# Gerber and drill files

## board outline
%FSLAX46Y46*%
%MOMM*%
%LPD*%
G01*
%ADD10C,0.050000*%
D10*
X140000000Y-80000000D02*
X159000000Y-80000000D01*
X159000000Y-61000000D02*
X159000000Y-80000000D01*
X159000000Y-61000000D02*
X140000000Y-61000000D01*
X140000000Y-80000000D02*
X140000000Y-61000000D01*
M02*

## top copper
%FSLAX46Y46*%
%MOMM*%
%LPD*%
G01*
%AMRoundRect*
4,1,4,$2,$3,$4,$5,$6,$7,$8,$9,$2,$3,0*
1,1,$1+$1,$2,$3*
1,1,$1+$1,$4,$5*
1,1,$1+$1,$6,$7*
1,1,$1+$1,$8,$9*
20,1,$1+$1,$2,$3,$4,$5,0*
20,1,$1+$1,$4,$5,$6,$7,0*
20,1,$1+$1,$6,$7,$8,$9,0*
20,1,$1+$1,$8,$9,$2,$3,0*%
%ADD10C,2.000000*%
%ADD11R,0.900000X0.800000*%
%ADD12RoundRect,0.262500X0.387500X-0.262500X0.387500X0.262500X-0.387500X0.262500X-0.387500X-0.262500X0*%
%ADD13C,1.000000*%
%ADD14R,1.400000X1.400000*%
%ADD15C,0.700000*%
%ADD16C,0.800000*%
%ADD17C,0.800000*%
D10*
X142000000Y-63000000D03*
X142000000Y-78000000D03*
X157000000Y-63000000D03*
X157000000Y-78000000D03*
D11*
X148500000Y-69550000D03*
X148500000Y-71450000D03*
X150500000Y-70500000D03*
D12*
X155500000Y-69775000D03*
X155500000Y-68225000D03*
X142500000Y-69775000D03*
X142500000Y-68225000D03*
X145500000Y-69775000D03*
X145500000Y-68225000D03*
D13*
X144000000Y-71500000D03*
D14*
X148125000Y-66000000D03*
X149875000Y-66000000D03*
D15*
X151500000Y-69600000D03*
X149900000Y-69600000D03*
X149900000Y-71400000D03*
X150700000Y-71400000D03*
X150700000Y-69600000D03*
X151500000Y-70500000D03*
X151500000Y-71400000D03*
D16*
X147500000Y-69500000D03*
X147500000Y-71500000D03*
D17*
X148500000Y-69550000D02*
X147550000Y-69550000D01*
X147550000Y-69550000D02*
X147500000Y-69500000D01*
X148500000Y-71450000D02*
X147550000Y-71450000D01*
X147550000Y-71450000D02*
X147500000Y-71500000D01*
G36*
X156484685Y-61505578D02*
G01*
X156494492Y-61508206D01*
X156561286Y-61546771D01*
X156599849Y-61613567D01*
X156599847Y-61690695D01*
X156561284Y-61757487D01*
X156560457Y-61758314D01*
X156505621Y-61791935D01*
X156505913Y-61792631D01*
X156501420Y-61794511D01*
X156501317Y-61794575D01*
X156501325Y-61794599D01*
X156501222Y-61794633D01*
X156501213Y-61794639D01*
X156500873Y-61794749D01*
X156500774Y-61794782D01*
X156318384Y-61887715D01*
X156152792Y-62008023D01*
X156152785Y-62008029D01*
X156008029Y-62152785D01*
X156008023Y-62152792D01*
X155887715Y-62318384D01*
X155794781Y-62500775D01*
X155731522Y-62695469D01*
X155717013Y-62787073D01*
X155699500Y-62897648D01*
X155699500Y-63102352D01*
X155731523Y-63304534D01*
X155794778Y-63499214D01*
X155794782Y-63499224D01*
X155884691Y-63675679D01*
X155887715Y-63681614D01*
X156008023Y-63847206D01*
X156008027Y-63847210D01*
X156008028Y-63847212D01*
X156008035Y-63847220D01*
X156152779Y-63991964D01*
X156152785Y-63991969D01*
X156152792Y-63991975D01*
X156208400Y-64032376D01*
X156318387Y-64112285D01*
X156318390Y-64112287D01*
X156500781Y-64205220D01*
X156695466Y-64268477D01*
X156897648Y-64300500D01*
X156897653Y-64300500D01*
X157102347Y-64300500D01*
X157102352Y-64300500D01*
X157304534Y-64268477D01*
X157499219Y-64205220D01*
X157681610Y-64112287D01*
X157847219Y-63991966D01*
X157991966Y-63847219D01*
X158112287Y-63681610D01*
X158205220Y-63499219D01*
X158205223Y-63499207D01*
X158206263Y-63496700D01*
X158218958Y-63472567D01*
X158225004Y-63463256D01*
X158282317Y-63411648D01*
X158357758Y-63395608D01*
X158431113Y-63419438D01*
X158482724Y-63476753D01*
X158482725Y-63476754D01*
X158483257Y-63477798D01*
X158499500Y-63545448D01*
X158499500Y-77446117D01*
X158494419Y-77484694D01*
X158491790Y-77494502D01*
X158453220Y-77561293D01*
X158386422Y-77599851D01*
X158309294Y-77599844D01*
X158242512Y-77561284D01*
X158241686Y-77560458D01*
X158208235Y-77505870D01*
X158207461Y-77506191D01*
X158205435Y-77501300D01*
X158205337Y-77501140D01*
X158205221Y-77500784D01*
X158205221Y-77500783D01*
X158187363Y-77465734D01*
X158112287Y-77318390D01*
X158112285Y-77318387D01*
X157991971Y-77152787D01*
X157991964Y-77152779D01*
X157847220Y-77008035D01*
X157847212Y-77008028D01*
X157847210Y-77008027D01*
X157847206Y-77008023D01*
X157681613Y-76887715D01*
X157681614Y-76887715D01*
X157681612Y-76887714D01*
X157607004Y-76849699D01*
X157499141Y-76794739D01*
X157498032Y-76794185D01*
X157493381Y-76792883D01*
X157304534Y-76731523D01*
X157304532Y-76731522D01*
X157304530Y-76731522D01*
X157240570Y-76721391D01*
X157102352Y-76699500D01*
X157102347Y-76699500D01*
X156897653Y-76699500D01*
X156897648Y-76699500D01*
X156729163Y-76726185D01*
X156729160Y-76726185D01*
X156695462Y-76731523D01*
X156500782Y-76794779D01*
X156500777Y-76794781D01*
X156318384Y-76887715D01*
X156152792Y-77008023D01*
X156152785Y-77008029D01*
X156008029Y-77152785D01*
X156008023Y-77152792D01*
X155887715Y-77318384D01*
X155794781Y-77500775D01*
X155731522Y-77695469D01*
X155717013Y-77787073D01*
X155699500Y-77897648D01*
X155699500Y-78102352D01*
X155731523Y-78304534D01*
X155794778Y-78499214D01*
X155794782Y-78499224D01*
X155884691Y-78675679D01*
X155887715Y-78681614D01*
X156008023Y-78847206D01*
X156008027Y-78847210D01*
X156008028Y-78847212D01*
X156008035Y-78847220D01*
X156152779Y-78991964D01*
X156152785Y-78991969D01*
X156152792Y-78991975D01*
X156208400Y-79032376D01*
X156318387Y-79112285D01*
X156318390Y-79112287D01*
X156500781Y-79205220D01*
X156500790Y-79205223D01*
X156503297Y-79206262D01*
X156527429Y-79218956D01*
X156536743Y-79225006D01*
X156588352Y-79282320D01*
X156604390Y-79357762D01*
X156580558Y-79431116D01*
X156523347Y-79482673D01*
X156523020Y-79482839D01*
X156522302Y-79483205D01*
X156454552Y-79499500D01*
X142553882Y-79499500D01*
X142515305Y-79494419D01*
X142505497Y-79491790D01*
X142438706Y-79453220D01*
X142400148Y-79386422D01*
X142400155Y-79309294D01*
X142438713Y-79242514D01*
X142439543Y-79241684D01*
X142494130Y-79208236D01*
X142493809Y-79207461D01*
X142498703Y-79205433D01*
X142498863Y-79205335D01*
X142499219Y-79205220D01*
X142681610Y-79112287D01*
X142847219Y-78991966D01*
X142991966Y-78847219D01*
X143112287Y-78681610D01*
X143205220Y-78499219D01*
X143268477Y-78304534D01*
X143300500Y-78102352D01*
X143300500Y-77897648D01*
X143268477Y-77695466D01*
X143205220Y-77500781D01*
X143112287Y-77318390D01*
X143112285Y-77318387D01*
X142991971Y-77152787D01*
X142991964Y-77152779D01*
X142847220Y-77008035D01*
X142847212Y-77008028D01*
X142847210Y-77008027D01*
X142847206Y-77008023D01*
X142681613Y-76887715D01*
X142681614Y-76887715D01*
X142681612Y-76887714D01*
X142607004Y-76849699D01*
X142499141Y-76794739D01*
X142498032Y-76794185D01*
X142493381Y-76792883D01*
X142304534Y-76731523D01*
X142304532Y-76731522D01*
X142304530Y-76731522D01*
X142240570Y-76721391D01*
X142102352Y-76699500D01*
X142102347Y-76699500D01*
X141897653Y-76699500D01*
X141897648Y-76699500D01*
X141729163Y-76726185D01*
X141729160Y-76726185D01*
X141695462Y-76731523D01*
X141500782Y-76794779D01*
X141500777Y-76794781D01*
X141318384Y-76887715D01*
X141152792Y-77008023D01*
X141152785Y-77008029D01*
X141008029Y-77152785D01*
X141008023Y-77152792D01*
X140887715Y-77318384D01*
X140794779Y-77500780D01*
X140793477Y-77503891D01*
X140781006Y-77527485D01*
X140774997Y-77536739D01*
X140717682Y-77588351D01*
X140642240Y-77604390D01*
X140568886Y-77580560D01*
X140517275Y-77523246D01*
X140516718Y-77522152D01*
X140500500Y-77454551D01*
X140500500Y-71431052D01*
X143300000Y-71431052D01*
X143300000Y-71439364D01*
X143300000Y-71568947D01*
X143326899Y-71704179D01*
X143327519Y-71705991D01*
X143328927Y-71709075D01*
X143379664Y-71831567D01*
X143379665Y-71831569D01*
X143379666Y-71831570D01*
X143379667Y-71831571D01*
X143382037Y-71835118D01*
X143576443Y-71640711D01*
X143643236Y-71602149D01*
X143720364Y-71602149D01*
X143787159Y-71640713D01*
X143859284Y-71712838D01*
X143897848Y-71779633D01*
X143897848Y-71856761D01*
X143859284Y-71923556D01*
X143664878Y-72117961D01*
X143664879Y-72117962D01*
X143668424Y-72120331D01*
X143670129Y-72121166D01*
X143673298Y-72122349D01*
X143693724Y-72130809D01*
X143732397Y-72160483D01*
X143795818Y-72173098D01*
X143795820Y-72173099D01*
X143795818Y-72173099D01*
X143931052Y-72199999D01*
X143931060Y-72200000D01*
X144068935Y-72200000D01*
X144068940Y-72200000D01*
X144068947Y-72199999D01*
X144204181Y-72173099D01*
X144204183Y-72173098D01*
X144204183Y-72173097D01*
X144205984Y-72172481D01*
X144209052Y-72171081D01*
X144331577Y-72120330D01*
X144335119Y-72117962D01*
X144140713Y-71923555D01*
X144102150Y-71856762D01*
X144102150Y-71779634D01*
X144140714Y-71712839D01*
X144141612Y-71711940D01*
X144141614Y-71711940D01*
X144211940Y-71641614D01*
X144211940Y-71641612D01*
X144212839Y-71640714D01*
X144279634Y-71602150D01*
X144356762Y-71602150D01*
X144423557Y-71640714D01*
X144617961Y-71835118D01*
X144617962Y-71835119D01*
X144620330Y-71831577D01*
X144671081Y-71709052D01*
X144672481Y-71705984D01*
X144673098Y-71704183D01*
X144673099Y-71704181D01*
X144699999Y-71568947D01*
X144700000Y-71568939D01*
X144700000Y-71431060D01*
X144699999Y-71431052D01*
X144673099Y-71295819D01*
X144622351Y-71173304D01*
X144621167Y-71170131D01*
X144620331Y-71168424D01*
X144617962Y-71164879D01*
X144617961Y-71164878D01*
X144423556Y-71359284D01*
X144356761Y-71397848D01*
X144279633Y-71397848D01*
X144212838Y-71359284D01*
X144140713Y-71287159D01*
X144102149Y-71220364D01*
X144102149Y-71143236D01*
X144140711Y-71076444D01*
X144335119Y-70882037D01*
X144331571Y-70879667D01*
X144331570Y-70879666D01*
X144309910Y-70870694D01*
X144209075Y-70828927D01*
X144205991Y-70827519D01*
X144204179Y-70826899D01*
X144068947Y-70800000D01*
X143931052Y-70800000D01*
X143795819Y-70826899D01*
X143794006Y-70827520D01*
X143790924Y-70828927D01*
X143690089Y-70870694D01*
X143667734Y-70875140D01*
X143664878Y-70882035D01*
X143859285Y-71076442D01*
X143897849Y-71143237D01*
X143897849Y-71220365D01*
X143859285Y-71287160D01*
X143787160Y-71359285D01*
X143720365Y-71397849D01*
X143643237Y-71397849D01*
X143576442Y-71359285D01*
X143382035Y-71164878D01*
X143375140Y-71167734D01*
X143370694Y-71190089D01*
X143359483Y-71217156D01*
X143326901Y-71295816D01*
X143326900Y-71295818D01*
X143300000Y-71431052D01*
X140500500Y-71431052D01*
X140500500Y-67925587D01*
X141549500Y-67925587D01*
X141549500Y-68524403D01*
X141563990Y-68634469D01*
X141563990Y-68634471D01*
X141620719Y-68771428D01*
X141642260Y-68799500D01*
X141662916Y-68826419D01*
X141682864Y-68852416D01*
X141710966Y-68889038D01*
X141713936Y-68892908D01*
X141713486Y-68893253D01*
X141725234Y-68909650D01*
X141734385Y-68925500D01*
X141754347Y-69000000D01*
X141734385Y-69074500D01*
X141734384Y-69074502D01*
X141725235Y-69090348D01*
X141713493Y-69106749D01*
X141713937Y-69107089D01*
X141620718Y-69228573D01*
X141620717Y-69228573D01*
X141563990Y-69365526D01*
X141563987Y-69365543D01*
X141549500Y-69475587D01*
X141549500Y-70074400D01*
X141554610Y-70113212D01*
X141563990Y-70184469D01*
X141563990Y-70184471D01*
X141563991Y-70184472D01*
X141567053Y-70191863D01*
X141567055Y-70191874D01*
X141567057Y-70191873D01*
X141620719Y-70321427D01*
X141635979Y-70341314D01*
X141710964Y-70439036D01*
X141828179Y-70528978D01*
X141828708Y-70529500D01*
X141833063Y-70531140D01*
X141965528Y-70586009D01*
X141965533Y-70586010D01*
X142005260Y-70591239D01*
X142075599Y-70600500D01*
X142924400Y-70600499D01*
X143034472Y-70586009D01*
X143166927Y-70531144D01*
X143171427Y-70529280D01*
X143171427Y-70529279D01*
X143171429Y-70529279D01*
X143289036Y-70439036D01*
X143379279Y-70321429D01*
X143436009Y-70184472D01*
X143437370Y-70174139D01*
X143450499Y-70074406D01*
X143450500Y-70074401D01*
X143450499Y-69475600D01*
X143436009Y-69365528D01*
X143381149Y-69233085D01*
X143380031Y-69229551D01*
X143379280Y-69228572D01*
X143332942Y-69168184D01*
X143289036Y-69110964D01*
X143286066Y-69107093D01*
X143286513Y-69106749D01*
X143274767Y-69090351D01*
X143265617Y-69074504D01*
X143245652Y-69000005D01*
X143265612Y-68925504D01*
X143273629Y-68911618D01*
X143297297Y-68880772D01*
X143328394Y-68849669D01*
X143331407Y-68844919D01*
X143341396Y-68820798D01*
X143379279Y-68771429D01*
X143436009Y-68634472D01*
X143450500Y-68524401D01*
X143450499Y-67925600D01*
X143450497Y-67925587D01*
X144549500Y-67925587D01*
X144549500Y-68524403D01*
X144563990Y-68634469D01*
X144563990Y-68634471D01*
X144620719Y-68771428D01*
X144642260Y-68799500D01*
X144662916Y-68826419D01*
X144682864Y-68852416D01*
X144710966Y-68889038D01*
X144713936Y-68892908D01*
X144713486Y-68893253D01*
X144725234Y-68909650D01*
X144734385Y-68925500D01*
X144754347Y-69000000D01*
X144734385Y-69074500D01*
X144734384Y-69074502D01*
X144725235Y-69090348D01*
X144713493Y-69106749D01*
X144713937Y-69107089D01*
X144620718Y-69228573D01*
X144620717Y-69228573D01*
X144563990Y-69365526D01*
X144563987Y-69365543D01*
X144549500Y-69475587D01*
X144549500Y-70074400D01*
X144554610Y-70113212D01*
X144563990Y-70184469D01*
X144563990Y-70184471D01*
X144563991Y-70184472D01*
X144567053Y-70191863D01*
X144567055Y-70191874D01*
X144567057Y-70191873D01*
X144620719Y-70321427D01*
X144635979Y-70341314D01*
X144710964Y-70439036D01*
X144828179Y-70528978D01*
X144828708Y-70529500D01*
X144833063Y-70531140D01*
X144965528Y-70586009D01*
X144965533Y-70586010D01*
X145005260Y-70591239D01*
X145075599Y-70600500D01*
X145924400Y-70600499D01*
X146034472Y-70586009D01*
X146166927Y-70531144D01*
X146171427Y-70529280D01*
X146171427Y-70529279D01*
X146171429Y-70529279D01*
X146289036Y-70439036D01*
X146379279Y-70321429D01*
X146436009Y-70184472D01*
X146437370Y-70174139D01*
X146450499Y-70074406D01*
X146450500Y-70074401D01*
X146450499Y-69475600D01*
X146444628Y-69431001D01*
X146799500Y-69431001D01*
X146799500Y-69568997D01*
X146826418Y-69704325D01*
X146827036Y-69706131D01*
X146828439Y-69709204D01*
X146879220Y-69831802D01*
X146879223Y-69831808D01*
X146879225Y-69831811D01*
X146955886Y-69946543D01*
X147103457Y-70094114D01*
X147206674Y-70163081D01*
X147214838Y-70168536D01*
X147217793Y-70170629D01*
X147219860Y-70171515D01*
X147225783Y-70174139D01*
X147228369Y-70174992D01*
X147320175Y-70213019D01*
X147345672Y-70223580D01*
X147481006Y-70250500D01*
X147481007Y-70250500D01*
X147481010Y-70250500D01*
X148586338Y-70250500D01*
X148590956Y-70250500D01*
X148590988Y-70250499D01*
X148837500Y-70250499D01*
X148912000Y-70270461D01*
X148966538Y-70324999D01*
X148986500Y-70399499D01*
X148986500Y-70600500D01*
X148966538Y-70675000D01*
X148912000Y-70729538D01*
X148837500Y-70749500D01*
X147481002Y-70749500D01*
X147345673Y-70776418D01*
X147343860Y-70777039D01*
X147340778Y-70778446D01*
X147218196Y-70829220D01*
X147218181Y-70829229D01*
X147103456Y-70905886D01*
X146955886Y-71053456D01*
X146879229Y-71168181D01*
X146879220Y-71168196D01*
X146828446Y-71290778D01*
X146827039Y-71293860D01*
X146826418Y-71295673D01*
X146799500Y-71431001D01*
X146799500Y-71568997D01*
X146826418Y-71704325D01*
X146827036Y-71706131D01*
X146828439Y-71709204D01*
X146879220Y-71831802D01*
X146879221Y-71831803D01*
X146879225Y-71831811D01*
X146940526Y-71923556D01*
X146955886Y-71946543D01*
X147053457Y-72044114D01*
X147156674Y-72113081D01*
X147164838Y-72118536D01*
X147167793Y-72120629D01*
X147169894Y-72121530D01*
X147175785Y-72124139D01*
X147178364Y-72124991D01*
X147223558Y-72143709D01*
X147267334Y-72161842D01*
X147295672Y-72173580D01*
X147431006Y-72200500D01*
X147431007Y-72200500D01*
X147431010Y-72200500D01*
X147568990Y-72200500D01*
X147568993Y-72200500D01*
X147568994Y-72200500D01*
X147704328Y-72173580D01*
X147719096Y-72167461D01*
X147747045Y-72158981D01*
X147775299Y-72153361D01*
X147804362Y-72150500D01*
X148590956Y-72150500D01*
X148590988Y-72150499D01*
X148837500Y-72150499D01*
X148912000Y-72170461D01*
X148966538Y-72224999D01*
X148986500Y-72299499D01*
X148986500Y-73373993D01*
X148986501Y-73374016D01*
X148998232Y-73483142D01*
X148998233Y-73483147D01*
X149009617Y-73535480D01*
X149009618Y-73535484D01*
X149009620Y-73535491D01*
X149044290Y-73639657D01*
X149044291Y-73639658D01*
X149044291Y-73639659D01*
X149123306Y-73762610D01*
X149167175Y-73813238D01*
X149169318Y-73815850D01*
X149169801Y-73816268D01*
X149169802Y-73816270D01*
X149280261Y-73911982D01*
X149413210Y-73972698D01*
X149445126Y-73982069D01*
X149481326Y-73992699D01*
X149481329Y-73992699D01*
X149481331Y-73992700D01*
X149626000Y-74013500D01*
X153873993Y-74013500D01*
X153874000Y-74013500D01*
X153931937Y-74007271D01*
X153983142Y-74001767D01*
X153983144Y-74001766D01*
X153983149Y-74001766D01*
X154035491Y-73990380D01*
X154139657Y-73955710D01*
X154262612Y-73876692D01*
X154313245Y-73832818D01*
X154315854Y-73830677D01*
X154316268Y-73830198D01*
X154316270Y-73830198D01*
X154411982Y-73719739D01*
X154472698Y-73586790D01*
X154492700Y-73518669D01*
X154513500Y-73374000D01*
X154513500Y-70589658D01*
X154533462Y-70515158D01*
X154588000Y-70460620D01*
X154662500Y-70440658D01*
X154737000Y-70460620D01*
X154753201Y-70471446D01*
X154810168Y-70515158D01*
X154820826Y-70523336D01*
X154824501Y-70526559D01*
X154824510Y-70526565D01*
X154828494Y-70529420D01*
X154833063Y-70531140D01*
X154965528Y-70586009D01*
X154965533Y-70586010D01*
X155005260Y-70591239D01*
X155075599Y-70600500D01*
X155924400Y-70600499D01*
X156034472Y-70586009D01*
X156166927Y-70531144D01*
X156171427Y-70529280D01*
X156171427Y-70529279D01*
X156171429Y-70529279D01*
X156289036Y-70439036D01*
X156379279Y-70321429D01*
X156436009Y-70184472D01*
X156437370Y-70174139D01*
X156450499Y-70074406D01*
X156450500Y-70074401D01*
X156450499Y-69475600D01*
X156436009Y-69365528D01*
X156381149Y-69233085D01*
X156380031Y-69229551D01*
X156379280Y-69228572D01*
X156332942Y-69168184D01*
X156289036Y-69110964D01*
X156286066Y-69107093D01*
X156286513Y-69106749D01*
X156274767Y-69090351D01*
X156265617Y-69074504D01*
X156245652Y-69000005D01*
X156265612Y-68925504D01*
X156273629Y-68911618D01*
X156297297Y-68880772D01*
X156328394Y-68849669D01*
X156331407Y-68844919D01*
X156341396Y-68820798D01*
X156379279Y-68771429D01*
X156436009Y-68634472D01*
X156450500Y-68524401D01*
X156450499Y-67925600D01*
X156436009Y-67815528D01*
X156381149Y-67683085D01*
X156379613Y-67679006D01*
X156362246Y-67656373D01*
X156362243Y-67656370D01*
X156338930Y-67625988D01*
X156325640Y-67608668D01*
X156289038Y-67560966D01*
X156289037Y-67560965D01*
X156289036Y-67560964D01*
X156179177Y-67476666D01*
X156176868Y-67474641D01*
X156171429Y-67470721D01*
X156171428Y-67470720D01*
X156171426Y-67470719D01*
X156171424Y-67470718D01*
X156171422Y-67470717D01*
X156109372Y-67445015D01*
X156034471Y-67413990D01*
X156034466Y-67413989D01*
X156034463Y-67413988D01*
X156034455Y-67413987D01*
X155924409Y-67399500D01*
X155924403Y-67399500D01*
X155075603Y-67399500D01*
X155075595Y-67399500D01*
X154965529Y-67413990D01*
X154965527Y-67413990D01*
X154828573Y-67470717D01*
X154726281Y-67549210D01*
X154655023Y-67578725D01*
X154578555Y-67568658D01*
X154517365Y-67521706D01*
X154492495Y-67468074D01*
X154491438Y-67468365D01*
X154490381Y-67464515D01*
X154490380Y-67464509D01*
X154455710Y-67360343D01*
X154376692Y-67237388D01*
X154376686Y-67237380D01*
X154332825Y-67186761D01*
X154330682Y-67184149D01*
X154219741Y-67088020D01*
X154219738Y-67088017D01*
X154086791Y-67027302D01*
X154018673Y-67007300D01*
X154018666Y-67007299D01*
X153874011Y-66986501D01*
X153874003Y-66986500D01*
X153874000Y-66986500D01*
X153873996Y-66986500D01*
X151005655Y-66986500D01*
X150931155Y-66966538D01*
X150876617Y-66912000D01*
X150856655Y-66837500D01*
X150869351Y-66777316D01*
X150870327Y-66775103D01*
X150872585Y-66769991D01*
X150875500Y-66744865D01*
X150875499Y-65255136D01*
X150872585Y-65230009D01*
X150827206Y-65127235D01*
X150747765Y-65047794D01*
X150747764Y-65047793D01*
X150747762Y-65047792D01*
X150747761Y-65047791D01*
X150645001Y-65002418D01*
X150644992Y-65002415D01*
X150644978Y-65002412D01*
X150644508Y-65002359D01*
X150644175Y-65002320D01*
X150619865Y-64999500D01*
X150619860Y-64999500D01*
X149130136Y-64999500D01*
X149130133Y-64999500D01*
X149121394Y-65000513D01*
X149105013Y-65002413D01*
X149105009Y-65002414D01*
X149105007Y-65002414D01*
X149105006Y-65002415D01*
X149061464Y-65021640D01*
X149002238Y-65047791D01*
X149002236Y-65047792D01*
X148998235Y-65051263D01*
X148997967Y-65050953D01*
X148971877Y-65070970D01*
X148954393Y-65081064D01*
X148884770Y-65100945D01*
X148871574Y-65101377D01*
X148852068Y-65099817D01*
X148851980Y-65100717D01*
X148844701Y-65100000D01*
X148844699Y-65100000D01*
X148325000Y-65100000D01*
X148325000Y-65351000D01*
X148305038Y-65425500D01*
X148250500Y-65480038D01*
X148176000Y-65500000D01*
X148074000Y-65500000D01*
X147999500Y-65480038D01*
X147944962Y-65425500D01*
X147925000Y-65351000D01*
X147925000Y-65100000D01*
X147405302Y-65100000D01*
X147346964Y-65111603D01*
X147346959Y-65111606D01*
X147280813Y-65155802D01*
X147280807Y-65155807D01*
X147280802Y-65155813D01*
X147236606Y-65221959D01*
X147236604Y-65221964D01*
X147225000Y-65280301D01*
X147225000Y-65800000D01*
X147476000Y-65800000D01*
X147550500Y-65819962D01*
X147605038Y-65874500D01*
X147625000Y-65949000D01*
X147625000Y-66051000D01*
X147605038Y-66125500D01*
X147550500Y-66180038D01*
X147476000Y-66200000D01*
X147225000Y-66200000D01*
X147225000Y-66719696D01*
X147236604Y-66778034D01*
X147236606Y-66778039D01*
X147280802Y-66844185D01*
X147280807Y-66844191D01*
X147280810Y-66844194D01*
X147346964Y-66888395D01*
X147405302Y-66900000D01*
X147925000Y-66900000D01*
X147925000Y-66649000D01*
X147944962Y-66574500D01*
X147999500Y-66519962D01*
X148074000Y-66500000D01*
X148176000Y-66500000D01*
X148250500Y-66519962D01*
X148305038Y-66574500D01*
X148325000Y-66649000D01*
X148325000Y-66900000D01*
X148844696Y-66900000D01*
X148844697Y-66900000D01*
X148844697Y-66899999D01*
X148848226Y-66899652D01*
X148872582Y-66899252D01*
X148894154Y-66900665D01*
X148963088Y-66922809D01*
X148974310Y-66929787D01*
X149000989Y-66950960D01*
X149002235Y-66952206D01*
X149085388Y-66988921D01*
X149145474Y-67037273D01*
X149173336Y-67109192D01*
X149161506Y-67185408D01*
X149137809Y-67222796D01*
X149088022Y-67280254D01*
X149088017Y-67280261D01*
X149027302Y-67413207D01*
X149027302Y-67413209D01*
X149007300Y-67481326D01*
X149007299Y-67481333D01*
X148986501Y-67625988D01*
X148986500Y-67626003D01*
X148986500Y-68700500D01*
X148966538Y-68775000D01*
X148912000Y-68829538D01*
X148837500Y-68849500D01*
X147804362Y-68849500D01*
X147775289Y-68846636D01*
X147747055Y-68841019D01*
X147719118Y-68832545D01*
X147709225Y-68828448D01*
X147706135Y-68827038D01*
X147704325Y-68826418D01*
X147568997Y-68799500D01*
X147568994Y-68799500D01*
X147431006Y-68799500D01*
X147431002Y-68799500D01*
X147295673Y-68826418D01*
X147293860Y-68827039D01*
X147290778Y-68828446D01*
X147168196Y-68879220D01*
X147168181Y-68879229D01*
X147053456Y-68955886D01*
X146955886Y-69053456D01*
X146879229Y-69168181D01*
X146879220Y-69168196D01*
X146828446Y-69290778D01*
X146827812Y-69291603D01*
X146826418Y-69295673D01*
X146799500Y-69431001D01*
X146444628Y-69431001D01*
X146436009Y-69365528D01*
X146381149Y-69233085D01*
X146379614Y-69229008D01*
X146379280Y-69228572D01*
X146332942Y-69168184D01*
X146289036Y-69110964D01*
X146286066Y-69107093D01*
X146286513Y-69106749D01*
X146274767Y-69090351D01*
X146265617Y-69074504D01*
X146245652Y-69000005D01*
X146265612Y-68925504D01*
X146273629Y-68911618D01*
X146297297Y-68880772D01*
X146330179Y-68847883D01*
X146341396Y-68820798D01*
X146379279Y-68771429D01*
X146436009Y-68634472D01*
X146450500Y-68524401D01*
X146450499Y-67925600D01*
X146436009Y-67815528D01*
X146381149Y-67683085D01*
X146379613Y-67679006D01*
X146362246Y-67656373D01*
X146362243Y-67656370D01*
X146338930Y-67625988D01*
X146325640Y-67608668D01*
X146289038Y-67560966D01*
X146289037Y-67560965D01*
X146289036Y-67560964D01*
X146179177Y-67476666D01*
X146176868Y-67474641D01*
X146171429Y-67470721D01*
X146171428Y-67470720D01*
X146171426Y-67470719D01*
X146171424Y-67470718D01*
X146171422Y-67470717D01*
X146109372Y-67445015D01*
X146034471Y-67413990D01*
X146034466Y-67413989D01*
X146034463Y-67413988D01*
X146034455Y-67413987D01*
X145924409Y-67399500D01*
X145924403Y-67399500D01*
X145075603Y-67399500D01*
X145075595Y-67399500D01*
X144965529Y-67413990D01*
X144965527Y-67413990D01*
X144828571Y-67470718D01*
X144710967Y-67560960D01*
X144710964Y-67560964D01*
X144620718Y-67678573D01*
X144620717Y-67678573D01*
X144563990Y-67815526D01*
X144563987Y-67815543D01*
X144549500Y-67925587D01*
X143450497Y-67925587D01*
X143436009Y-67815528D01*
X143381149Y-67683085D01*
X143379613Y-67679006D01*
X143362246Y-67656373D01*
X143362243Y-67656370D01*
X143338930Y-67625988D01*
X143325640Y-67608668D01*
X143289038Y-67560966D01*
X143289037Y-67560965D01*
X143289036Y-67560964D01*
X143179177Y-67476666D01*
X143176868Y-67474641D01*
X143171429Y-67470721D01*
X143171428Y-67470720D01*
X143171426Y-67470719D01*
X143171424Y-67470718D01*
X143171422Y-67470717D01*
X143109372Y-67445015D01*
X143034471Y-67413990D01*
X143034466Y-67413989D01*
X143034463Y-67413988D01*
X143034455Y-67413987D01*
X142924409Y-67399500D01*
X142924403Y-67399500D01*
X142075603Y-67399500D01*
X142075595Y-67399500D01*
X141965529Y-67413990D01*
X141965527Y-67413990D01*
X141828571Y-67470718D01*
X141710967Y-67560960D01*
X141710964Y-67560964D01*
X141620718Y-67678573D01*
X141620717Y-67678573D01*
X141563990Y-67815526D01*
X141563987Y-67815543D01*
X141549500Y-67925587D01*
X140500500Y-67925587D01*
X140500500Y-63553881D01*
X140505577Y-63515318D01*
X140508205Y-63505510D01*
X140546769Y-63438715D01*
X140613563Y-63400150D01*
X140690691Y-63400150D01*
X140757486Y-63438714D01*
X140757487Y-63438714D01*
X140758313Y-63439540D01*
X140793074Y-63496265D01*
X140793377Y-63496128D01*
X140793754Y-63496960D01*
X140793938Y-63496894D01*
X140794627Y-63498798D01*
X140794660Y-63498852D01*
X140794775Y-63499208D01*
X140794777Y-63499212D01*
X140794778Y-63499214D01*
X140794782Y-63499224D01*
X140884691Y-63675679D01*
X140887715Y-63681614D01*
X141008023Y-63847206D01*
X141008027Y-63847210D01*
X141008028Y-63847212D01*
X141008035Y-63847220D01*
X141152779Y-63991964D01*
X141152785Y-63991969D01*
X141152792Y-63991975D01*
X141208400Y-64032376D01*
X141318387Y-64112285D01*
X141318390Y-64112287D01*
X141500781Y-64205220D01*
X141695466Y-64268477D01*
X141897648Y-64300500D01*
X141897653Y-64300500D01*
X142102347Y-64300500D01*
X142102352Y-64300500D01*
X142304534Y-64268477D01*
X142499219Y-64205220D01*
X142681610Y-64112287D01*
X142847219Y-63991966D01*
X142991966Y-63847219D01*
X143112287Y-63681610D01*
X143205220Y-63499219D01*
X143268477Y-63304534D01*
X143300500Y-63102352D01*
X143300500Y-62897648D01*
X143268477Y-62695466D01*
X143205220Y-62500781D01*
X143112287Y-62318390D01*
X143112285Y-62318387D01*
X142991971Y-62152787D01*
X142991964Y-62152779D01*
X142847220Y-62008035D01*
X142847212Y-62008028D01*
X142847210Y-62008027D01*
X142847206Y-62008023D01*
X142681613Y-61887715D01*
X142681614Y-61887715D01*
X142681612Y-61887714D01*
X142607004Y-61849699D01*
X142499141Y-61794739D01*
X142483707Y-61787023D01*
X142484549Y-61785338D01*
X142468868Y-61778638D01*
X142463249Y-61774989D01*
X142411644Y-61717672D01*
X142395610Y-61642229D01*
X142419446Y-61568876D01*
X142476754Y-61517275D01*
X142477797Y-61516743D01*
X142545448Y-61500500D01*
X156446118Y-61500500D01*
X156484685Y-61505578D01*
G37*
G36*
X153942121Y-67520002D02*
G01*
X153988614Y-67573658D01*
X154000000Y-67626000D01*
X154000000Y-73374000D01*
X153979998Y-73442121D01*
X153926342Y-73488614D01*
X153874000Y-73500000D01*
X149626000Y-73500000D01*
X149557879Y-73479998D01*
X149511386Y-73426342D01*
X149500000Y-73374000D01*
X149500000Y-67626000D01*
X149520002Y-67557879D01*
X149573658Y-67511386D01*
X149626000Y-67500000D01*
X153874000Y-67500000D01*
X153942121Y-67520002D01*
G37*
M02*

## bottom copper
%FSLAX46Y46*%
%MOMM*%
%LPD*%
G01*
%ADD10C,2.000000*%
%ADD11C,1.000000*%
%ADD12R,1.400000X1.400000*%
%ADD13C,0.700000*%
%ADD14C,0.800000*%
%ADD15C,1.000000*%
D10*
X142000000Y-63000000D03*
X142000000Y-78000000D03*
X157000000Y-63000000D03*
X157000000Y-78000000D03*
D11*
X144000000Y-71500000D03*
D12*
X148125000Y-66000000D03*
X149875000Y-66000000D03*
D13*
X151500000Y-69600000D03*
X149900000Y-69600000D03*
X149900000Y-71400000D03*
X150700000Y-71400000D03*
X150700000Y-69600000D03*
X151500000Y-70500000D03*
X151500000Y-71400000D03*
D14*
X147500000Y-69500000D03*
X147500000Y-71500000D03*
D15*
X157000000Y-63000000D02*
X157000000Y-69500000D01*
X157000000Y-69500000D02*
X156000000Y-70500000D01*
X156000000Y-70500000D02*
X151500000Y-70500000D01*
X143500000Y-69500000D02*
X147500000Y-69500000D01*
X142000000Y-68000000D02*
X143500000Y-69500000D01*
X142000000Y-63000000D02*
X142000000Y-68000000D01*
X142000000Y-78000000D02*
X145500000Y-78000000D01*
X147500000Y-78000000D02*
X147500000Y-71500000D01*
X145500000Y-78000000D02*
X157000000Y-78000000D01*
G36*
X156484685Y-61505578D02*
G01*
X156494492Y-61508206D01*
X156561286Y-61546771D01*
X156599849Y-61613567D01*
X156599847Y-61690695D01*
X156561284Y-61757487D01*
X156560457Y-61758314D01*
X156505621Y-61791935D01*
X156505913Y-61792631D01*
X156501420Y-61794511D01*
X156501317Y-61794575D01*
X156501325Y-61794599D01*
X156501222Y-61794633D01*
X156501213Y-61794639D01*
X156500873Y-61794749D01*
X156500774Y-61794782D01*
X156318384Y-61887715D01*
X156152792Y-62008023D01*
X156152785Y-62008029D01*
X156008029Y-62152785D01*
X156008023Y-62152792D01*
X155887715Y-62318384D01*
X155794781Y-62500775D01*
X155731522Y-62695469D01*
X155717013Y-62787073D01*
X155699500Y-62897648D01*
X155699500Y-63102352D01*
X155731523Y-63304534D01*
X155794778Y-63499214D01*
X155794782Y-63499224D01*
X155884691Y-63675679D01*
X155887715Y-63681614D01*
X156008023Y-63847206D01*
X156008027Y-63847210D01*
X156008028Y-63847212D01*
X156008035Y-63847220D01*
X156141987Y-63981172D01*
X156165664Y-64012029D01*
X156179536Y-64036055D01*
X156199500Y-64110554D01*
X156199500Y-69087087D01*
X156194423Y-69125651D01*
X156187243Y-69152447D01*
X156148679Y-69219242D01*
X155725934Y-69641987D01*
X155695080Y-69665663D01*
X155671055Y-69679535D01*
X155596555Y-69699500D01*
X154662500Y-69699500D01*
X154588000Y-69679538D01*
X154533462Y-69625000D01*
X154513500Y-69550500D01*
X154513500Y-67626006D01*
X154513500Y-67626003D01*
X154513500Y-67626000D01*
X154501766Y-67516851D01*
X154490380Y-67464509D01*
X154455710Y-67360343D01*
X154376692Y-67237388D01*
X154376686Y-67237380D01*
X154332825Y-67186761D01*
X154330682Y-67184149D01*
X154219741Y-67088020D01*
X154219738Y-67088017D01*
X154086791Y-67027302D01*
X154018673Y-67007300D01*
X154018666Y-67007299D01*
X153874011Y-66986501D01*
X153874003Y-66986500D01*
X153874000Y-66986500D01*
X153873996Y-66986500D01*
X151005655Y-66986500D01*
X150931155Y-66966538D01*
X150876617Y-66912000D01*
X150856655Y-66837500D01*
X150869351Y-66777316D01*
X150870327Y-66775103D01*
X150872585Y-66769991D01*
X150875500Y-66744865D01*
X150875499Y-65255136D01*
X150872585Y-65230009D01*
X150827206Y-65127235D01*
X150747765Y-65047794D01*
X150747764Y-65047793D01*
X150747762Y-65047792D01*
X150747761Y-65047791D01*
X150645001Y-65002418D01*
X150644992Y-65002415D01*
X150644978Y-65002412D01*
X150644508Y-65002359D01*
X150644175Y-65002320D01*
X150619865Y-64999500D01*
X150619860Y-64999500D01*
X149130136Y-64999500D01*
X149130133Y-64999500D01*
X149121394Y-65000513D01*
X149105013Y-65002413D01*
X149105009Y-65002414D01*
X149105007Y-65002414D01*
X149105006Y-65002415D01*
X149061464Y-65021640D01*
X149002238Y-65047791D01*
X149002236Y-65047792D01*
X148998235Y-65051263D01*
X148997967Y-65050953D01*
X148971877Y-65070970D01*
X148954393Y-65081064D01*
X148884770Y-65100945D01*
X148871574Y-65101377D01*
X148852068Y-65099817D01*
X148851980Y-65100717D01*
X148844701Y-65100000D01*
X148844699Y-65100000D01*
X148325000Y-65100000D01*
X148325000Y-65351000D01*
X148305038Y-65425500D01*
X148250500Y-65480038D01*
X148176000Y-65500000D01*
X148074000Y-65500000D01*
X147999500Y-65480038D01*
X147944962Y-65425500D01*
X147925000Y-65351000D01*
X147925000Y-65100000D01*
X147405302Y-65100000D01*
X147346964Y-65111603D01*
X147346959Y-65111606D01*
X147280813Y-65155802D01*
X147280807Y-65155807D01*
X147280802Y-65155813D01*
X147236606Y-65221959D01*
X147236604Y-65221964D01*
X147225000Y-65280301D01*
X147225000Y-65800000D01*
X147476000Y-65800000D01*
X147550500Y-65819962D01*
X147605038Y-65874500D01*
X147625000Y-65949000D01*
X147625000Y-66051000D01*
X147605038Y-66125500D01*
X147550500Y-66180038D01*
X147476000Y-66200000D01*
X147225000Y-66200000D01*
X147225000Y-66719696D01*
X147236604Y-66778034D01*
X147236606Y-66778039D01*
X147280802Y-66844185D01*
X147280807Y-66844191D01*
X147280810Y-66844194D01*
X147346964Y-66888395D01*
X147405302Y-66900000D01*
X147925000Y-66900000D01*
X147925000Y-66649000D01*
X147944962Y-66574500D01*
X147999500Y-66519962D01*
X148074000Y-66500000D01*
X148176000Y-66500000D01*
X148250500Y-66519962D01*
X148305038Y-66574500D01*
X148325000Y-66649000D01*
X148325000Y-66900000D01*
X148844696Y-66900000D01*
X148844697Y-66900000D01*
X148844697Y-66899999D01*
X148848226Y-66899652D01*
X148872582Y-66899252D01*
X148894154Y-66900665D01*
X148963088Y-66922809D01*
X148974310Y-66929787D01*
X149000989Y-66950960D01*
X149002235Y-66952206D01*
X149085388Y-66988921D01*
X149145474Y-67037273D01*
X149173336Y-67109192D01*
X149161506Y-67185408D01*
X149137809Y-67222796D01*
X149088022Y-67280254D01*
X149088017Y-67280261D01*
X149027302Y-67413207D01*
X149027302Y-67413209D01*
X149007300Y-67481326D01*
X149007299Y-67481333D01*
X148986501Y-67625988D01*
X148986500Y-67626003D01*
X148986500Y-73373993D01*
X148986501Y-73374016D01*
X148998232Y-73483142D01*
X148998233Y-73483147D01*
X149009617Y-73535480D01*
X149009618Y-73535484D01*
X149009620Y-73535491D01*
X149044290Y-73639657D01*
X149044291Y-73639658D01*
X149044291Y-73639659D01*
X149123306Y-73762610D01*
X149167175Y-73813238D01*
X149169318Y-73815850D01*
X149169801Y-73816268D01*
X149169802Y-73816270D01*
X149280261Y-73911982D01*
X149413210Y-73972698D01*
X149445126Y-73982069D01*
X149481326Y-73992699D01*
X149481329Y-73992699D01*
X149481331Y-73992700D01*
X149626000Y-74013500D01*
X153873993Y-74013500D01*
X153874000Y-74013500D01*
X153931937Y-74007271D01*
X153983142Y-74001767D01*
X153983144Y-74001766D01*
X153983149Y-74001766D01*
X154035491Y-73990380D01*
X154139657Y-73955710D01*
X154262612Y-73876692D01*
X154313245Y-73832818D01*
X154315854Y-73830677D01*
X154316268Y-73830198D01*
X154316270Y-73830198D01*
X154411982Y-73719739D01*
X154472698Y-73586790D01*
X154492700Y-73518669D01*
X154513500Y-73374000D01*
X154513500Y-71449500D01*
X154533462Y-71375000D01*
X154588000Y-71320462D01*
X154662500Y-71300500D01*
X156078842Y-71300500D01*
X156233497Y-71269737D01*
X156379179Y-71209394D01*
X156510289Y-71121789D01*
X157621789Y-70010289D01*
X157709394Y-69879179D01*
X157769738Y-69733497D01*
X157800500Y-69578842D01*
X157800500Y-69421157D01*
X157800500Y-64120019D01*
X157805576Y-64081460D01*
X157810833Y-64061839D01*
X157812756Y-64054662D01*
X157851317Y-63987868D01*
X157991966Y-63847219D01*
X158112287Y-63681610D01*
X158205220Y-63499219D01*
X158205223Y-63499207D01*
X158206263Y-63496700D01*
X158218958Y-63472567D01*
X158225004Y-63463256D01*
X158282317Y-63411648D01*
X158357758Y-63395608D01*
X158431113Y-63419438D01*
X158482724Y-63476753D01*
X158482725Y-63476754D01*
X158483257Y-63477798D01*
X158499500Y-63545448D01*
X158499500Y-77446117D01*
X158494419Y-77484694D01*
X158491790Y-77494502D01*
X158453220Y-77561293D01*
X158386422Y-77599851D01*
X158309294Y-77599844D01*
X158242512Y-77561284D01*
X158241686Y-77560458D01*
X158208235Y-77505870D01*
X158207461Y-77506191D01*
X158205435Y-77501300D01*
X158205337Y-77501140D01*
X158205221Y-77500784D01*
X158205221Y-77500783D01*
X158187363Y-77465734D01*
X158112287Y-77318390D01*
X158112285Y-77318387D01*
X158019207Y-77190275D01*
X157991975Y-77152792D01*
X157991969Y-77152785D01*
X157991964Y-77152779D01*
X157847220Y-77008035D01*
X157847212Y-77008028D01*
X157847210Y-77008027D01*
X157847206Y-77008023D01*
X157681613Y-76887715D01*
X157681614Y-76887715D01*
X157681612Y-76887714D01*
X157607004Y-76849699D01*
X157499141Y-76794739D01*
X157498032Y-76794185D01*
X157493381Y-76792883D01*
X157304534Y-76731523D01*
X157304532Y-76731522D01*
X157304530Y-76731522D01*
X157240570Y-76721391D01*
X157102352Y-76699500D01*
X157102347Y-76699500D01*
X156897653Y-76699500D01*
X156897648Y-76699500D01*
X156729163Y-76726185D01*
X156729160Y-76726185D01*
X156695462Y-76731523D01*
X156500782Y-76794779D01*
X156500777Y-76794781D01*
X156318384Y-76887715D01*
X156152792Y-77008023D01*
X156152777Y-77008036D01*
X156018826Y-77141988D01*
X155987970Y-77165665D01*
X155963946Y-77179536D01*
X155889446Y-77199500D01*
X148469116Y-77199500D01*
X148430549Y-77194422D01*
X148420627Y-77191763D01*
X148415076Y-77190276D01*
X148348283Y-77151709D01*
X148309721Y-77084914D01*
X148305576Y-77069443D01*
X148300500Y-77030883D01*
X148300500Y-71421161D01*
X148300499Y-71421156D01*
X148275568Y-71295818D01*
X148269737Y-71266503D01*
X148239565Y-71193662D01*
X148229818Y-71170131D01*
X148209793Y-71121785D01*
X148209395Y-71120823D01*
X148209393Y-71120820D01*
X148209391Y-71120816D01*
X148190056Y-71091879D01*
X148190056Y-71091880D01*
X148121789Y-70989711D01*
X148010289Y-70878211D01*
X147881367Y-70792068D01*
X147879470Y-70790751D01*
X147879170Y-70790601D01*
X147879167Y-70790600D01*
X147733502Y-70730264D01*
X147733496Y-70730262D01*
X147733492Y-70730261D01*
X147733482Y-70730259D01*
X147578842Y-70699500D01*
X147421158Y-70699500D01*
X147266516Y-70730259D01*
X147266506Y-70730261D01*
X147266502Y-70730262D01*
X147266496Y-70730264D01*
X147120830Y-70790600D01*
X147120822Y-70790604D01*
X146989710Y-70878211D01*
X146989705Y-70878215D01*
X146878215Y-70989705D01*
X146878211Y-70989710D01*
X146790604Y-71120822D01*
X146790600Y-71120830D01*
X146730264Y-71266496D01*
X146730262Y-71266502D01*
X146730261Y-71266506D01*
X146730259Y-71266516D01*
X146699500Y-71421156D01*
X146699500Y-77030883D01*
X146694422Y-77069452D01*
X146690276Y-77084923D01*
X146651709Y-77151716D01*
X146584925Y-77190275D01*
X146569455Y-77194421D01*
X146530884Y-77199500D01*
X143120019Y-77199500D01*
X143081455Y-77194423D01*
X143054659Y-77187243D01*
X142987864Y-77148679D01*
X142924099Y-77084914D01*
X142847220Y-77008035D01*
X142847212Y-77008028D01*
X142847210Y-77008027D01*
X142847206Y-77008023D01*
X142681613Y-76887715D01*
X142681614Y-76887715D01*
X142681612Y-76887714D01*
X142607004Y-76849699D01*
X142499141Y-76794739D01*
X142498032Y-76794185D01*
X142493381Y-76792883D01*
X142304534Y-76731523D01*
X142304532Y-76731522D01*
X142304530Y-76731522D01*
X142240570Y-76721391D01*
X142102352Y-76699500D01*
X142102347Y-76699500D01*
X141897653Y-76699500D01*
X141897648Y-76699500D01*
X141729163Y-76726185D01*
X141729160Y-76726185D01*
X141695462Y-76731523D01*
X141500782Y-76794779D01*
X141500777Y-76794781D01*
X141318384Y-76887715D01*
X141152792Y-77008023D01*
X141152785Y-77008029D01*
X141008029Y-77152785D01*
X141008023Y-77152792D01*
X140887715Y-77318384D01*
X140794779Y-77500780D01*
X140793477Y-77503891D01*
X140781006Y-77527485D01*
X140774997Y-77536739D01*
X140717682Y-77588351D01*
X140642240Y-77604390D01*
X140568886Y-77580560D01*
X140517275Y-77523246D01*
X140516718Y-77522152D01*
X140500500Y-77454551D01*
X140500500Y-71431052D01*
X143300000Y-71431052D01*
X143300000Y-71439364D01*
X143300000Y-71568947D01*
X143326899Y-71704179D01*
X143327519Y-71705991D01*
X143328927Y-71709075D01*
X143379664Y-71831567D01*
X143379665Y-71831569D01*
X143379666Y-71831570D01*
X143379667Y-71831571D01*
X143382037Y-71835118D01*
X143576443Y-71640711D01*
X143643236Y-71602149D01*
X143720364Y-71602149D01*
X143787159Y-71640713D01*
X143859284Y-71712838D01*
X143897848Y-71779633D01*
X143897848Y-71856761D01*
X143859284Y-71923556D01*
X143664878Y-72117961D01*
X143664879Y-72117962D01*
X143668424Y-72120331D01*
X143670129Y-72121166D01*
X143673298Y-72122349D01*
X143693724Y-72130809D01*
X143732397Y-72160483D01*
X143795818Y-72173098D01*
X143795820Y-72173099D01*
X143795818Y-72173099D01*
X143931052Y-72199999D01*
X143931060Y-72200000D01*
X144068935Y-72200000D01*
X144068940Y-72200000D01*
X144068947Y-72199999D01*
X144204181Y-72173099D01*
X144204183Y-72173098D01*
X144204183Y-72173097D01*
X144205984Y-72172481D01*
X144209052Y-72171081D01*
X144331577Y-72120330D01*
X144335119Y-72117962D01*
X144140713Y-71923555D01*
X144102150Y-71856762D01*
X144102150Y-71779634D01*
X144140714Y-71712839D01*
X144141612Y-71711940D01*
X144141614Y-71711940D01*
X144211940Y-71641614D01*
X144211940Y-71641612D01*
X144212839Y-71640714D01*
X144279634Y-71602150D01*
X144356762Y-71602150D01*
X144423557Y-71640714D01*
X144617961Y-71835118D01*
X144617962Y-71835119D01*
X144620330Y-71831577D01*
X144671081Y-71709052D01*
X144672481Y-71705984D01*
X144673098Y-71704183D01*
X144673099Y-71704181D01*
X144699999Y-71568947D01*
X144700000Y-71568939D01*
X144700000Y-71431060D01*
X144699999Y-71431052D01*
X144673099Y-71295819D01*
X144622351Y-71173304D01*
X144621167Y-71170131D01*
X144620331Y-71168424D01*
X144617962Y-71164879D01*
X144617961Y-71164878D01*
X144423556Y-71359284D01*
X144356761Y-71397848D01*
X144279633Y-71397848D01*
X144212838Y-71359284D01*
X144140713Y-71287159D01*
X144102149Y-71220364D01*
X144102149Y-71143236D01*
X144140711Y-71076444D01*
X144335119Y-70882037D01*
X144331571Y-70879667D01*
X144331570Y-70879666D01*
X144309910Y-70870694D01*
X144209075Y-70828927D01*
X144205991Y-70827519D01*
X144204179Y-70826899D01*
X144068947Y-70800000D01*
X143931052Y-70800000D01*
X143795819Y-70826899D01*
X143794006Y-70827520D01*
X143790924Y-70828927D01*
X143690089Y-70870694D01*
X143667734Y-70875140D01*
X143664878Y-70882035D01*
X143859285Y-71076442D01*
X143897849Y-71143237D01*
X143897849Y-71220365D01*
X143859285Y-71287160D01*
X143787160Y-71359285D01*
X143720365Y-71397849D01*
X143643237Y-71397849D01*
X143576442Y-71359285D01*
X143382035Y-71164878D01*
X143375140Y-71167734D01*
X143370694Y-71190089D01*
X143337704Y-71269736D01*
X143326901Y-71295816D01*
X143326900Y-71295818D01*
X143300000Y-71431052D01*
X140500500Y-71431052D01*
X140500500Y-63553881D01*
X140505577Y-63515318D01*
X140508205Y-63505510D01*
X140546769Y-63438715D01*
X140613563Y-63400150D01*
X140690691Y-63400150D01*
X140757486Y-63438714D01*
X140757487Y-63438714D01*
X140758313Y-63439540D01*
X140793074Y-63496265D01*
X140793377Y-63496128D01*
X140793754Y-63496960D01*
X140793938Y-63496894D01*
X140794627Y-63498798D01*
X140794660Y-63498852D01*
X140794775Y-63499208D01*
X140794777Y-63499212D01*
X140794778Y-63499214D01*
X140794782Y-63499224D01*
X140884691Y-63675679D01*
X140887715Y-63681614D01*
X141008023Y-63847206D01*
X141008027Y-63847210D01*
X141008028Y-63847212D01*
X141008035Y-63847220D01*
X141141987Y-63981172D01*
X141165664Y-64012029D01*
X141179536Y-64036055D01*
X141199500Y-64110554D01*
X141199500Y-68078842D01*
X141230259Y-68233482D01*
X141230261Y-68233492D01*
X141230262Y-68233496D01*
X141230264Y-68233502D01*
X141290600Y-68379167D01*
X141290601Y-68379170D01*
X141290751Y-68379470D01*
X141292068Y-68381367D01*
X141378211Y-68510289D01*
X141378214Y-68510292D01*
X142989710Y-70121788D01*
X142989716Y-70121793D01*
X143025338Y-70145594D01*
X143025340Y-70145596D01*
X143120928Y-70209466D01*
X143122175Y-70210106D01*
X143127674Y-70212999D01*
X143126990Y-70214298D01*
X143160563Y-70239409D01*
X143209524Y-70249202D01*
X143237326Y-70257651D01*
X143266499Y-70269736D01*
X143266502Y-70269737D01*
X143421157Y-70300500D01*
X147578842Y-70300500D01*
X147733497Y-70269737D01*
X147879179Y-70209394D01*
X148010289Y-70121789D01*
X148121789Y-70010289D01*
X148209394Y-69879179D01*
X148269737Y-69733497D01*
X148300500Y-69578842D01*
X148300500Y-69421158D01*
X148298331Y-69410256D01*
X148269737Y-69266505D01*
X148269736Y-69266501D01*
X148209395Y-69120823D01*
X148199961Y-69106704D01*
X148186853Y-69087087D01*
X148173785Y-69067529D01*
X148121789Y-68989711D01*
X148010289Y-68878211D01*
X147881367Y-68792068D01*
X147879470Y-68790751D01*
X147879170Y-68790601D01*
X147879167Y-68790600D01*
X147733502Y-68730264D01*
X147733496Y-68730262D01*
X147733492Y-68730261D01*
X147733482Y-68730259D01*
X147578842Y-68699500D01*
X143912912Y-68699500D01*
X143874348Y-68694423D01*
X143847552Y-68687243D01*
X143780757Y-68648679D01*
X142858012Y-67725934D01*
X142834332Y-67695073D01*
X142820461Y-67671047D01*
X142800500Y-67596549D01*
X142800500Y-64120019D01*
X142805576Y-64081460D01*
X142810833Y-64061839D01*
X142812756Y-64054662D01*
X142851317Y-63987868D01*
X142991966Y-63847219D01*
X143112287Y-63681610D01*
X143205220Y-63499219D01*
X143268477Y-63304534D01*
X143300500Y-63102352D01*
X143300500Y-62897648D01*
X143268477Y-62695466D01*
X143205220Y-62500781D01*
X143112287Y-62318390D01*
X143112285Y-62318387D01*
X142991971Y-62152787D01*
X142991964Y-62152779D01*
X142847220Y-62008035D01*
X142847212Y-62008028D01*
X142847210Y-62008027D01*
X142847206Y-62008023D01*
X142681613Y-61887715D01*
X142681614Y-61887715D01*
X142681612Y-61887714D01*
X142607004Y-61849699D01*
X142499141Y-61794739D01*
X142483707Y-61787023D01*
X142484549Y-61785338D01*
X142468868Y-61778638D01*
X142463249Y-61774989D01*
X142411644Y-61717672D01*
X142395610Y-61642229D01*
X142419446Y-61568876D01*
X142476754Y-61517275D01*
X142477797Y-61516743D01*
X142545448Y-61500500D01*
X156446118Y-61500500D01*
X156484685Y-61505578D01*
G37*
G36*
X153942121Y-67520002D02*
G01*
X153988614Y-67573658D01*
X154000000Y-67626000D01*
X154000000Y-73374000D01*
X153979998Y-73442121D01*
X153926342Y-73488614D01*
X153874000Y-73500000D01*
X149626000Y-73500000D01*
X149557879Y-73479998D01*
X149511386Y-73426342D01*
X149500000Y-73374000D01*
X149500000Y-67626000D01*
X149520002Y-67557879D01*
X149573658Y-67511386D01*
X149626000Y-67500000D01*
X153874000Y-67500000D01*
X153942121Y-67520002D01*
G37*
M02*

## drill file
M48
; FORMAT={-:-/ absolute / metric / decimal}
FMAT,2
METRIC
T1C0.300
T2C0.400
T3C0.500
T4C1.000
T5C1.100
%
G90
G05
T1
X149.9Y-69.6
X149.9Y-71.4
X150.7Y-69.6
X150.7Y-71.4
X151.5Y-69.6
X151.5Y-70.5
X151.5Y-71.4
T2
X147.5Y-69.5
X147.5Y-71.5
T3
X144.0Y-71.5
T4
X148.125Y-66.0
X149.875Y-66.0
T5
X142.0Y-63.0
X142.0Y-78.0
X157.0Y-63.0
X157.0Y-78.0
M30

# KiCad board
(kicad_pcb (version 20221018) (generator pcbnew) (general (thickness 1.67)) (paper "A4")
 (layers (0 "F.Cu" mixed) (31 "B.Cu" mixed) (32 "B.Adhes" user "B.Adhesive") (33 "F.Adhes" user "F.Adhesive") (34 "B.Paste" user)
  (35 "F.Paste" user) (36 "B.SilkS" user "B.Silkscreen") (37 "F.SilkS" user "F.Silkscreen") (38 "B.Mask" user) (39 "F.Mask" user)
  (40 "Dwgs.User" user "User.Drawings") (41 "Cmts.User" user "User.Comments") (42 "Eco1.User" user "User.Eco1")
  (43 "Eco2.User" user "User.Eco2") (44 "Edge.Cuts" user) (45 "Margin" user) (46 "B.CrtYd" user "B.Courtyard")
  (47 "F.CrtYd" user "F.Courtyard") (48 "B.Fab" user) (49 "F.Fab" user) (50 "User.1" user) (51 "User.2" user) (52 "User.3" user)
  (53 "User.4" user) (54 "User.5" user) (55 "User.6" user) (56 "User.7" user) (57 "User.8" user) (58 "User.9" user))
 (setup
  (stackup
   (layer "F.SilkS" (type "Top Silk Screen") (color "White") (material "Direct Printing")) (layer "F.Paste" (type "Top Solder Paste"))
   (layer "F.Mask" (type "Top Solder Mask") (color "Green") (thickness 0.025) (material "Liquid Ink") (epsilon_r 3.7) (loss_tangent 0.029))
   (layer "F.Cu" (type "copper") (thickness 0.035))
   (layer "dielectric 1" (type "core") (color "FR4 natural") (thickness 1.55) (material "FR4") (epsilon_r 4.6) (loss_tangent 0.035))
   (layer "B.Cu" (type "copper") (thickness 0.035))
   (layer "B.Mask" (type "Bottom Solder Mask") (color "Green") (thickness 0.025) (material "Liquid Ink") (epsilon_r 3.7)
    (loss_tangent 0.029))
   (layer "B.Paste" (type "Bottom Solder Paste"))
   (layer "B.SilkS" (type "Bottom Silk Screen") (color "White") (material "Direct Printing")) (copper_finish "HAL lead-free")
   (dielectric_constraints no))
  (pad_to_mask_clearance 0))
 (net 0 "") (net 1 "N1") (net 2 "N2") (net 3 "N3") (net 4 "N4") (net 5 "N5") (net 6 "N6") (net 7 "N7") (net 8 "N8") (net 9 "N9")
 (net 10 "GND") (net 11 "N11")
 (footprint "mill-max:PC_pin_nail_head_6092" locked (layer "F.Cu") (at 142 63)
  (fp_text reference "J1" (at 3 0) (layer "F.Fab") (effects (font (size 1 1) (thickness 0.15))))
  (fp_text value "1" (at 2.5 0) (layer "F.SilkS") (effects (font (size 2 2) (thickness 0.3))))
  (pad "1" thru_hole circle locked (at 0 0) (size 2 2) (drill 1.1) (layers "*.Cu" "*.Mask") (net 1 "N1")))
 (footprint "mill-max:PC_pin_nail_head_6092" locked (layer "F.Cu") (at 142 78)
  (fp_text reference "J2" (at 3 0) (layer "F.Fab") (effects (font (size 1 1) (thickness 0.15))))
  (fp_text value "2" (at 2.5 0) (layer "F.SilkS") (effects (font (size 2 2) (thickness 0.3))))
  (pad "1" thru_hole circle locked (at 0 0) (size 2 2) (drill 1.1) (layers "*.Cu" "*.Mask") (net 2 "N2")))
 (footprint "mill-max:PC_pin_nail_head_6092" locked (layer "F.Cu") (at 157 63)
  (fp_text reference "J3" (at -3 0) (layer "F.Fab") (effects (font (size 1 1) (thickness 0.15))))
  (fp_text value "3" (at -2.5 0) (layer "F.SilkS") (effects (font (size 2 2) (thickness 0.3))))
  (pad "1" thru_hole circle locked (at 0 0) (size 2 2) (drill 1.1) (layers "*.Cu" "*.Mask") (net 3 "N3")))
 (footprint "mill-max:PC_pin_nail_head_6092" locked (layer "F.Cu") (at 157 78)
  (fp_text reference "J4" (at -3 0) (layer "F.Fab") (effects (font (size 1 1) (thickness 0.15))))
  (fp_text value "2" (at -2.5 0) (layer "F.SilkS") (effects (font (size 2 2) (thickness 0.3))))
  (pad "1" thru_hole circle locked (at 0 0) (size 2 2) (drill 1.1) (layers "*.Cu" "*.Mask") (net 2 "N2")))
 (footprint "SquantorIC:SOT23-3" (layer "F.Cu") (at 149.5 70.5)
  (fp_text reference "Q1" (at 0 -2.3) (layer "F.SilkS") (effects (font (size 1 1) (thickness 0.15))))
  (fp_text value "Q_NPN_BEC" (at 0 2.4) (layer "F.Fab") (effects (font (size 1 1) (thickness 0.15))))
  (pad "1" smd rect (at -1 -0.95 270) (size 0.8 0.9) (layers "F.Cu" "F.Paste" "F.Mask") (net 1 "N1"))
  (pad "2" smd rect (at -1 0.95 270) (size 0.8 0.9) (layers "F.Cu" "F.Paste" "F.Mask") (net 2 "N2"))
  (pad "3" smd rect (at 1 0 270) (size 0.8 0.9) (layers "F.Cu" "F.Paste" "F.Mask") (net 3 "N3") (zone_connect 2)))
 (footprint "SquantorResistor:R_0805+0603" (layer "F.Cu") (at 155.5 69 90)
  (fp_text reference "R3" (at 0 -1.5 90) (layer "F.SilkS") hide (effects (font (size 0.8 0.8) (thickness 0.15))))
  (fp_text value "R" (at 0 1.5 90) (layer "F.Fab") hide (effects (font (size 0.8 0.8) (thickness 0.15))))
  (pad "1" smd roundrect (at -0.775 0 90) (size 1.05 1.3) (layers "F.Cu" "F.Paste" "F.Mask") (roundrect_rratio 0.25) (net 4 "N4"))
  (pad "2" smd roundrect (at 0.775 0 90) (size 1.05 1.3) (layers "F.Cu" "F.Paste" "F.Mask") (roundrect_rratio 0.25) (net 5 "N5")))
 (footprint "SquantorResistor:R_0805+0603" (layer "F.Cu") (at 142.5 69 90)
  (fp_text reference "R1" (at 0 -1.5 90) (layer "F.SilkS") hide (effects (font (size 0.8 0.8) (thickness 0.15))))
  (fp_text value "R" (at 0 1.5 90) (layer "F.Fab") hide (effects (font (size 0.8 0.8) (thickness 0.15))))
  (pad "1" smd roundrect (at -0.775 0 90) (size 1.05 1.3) (layers "F.Cu" "F.Paste" "F.Mask") (roundrect_rratio 0.25) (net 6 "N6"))
  (pad "2" smd roundrect (at 0.775 0 90) (size 1.05 1.3) (layers "F.Cu" "F.Paste" "F.Mask") (roundrect_rratio 0.25) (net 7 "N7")))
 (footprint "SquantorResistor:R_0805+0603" (layer "F.Cu") (at 145.5 69 90)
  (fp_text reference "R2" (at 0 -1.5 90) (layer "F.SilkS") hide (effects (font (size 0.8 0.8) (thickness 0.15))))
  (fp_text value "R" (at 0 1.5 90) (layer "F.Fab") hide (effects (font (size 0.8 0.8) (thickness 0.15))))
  (pad "1" smd roundrect (at -0.775 0 90) (size 1.05 1.3) (layers "F.Cu" "F.Paste" "F.Mask") (roundrect_rratio 0.25) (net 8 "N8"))
  (pad "2" smd roundrect (at 0.775 0 90) (size 1.05 1.3) (layers "F.Cu" "F.Paste" "F.Mask") (roundrect_rratio 0.25) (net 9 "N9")))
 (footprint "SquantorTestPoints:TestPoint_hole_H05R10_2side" (layer "F.Cu") (at 144 71.5)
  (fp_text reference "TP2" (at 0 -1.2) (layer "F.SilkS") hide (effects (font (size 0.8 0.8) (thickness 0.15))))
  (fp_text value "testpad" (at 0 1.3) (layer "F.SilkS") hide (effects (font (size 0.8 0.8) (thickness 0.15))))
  (pad "1" thru_hole circle (at 0 0) (size 1 1) (drill 0.5) (layers "*.Cu" "*.Mask") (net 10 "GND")))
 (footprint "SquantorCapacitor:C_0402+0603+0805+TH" (layer "F.Cu") (at 149 66)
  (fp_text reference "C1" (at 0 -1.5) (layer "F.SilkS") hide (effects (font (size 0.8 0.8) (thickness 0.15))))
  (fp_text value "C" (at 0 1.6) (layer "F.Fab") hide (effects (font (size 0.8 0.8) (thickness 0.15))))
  (pad "1" thru_hole rect (at -0.875 0) (size 1.4 1.4) (drill 1) (layers "*.Cu" "*.Mask") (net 10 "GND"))
  (pad "2" thru_hole rect (at 0.875 0) (size 1.4 1.4) (drill 1) (layers "*.Cu" "*.Mask") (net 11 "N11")))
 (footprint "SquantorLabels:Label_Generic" (layer "B.Cu") (at 157.25 71.5 90)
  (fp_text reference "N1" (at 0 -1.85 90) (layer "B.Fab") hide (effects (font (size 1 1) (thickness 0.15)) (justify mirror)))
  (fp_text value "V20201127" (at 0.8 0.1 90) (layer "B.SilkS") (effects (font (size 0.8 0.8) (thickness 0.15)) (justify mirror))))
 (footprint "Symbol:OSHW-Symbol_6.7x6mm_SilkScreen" (layer "B.Cu") (at 153.75 70.5 -90)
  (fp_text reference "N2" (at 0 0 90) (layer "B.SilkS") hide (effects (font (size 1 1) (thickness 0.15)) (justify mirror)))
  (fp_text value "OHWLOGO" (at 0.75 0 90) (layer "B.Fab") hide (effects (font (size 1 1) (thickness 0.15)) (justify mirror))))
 (gr_line (start 140 80) (end 159 80) (stroke (width 0.05) (type solid)) (layer "Edge.Cuts"))
 (gr_line (start 159 61) (end 159 80) (stroke (width 0.05) (type solid)) (layer "Edge.Cuts"))
 (gr_line (start 159 61) (end 140 61) (stroke (width 0.05) (type solid)) (layer "Edge.Cuts"))
 (gr_line (start 140 80) (end 140 61) (stroke (width 0.05) (type solid)) (layer "Edge.Cuts"))
 (via (at 151.5 69.6) (size 0.7) (drill 0.3) (layers "F.Cu" "B.Cu") (free) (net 3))
 (via (at 149.9 69.6) (size 0.7) (drill 0.3) (layers "F.Cu" "B.Cu") (free) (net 3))
 (via (at 149.9 71.4) (size 0.7) (drill 0.3) (layers "F.Cu" "B.Cu") (free) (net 3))
 (via (at 150.7 71.4) (size 0.7) (drill 0.3) (layers "F.Cu" "B.Cu") (free) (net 3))
 (via (at 150.7 69.6) (size 0.7) (drill 0.3) (layers "F.Cu" "B.Cu") (free) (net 3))
 (via (at 151.5 70.5) (size 0.7) (drill 0.3) (layers "F.Cu" "B.Cu") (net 3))
 (via (at 151.5 71.4) (size 0.7) (drill 0.3) (layers "F.Cu" "B.Cu") (free) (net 3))
 (segment (start 157 63) (end 157 69.5) (width 1) (layer "B.Cu") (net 3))
 (segment (start 157 69.5) (end 156 70.5) (width 1) (layer "B.Cu") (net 3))
 (segment (start 156 70.5) (end 151.5 70.5) (width 1) (layer "B.Cu") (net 3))
 (segment (start 148.5 69.55) (end 147.55 69.55) (width 0.8) (layer "F.Cu") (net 1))
 (segment (start 147.55 69.55) (end 147.5 69.5) (width 0.8) (layer "F.Cu") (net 1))
 (via (at 147.5 69.5) (size 0.8) (drill 0.4) (layers "F.Cu" "B.Cu") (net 1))
 (segment (start 143.5 69.5) (end 147.5 69.5) (width 1) (layer "B.Cu") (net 1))
 (segment (start 142 68) (end 143.5 69.5) (width 1) (layer "B.Cu") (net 1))
 (segment (start 142 63) (end 142 68) (width 1) (layer "B.Cu") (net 1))
 (segment (start 148.5 71.45) (end 147.55 71.45) (width 0.8) (layer "F.Cu") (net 2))
 (segment (start 147.55 71.45) (end 147.5 71.5) (width 0.8) (layer "F.Cu") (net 2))
 (via (at 147.5 71.5) (size 0.8) (drill 0.4) (layers "F.Cu" "B.Cu") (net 2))
 (segment (start 142 78) (end 145.5 78) (width 1) (layer "B.Cu") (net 2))
 (segment (start 147.5 78) (end 147.5 71.5) (width 1) (layer "B.Cu") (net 2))
 (segment (start 145.5 78) (end 157 78) (width 1) (layer "B.Cu") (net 2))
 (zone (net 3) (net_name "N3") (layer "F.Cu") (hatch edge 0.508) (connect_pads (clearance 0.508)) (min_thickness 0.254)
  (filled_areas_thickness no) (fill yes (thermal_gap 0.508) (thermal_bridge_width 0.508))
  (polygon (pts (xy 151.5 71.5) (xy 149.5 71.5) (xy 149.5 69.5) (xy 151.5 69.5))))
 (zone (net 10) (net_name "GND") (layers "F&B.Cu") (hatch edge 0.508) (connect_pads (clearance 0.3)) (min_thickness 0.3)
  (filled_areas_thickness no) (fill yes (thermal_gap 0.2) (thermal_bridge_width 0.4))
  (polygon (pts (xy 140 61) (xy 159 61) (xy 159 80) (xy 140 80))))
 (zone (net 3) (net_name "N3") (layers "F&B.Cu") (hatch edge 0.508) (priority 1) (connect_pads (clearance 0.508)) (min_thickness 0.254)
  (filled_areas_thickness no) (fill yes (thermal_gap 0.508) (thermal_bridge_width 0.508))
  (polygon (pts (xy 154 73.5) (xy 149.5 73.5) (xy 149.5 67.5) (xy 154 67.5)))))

